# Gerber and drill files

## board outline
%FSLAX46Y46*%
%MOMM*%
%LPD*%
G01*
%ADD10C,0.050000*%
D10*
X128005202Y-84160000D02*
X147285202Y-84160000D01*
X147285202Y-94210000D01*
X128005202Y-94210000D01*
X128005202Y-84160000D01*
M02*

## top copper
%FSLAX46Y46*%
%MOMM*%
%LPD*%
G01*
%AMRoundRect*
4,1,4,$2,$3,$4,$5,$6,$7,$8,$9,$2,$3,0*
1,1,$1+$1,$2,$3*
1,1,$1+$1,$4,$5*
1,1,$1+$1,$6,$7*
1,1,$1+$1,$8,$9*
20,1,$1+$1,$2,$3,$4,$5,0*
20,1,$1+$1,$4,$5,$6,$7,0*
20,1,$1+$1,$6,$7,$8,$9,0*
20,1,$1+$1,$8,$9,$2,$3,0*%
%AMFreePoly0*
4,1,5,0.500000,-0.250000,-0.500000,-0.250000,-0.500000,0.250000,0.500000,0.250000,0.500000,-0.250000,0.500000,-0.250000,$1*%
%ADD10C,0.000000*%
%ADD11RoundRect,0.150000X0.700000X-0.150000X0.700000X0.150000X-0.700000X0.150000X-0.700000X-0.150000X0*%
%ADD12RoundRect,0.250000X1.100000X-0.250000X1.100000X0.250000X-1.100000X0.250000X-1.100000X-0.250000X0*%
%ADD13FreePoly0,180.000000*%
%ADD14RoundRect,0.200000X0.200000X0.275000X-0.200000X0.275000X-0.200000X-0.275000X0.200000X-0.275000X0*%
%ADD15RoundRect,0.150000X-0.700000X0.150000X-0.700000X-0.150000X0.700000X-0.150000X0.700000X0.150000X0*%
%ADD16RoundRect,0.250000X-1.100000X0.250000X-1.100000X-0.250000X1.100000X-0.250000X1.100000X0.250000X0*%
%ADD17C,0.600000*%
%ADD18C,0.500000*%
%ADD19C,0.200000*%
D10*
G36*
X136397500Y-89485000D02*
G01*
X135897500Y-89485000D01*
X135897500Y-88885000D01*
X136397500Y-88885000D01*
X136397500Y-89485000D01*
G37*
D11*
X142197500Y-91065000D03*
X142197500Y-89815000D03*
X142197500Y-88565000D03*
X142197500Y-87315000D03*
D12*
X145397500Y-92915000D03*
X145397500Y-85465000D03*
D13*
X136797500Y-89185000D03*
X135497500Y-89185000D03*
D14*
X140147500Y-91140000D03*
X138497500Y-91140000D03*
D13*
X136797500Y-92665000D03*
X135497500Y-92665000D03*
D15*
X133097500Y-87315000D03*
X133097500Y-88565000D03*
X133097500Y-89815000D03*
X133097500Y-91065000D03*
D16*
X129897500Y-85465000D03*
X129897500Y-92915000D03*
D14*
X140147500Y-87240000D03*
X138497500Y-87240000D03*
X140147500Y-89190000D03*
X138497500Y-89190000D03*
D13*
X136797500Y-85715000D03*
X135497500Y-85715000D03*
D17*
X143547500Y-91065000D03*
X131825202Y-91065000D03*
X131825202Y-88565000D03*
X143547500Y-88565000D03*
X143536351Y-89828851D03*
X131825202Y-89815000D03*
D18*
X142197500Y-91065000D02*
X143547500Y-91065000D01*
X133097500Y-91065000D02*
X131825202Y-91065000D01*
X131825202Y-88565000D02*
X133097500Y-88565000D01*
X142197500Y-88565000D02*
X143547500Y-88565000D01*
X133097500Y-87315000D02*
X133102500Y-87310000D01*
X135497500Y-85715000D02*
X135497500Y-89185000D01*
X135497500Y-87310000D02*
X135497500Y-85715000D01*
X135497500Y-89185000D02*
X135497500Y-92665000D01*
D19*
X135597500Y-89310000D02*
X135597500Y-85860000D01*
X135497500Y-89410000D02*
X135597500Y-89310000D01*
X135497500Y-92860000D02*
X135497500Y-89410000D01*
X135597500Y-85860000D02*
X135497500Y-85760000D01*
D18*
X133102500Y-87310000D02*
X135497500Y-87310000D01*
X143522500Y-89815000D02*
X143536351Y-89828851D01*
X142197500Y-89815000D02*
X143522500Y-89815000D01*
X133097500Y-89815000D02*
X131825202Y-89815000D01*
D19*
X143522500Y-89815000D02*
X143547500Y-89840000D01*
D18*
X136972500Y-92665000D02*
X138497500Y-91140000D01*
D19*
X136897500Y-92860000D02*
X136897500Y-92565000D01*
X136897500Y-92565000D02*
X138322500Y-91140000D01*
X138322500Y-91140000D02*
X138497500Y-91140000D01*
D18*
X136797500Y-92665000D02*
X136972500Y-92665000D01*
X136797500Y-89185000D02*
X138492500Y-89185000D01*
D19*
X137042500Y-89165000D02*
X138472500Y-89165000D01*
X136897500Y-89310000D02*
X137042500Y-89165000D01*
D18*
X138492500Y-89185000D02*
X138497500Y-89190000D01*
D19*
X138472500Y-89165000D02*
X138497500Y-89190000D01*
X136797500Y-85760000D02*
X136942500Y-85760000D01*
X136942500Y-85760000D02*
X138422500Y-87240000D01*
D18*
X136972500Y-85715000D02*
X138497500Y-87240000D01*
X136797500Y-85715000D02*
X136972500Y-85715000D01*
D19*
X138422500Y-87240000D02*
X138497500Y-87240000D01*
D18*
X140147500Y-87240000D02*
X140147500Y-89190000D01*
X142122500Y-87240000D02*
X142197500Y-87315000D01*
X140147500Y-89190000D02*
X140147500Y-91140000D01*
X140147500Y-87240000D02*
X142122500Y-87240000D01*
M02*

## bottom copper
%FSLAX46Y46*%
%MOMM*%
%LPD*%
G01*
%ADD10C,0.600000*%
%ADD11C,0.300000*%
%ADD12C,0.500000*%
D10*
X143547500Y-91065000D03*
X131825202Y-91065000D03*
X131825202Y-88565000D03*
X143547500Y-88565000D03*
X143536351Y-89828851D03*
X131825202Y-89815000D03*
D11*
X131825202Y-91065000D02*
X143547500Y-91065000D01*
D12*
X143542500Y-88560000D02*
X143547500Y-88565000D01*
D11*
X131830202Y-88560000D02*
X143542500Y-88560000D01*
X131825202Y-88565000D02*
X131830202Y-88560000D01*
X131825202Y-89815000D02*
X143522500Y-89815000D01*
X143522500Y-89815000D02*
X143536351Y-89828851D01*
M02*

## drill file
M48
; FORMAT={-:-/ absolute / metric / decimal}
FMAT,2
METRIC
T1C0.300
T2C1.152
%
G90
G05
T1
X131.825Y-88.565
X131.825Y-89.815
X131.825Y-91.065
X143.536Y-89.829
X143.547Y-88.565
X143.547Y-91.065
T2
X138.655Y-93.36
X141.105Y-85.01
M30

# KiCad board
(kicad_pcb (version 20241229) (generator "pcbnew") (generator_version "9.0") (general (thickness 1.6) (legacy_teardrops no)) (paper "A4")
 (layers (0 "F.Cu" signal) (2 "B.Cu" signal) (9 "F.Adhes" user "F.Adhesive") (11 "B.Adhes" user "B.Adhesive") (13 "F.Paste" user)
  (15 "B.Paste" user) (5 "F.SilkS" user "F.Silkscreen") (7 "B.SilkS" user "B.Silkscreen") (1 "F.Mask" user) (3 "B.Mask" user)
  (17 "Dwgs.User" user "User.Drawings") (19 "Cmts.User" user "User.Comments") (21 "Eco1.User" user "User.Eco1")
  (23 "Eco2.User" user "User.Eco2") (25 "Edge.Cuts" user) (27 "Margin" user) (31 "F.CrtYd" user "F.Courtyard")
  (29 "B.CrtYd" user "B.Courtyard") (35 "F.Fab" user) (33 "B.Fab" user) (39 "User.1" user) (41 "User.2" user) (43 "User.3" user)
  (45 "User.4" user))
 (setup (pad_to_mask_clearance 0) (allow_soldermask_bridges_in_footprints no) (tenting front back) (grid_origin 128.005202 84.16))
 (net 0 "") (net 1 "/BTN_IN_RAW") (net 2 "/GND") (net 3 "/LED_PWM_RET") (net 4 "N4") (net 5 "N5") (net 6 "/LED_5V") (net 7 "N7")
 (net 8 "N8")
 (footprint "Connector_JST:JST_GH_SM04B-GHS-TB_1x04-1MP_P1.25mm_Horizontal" (layer "F.Cu") (at 144.0475 89.19 90)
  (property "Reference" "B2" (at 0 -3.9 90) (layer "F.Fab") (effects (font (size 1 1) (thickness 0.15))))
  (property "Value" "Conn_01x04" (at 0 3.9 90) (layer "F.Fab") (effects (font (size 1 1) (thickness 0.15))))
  (pad "1" smd roundrect (at -1.875 -1.85 90) (size 0.6 1.7) (layers "F.Cu" "F.Mask" "F.Paste") (roundrect_rratio 0.25)
   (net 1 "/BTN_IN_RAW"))
  (pad "2" smd roundrect (at -0.625 -1.85 90) (size 0.6 1.7) (layers "F.Cu" "F.Mask" "F.Paste") (roundrect_rratio 0.25) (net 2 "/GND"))
  (pad "3" smd roundrect (at 0.625 -1.85 90) (size 0.6 1.7) (layers "F.Cu" "F.Mask" "F.Paste") (roundrect_rratio 0.25)
   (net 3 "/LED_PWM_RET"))
  (pad "4" smd roundrect (at 1.875 -1.85 90) (size 0.6 1.7) (layers "F.Cu" "F.Mask" "F.Paste") (roundrect_rratio 0.25) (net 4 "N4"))
  (pad "MP" smd roundrect (at -3.725 1.35 90) (size 1 2.7) (layers "F.Cu" "F.Mask" "F.Paste") (roundrect_rratio 0.25))
  (pad "MP" smd roundrect (at 3.725 1.35 90) (size 1 2.7) (layers "F.Cu" "F.Mask" "F.Paste") (roundrect_rratio 0.25)))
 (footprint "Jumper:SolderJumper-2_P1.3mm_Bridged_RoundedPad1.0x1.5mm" (layer "F.Cu") (at 136.1475 89.185 180)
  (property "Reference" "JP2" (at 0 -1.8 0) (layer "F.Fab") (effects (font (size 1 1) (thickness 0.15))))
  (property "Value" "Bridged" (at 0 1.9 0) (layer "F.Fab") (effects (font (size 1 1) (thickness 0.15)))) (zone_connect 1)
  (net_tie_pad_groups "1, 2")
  (fp_poly (pts (xy 0.25 -0.3) (xy -0.25 -0.3) (xy -0.25 0.3) (xy 0.25 0.3)) (stroke (width 0) (type solid)) (fill yes) (layer "F.Cu"))
  (pad "1" smd custom (at -0.65 0 180) (size 1 0.5) (layers "F.Cu" "F.Mask") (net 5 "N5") (zone_connect 2) (thermal_bridge_angle 45)
   (options (clearance outline) (anchor rect)) (primitives))
  (pad "2" smd custom (at 0.65 0 180) (size 1 0.5) (layers "F.Cu" "F.Mask") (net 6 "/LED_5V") (zone_connect 2) (thermal_bridge_angle 45)
   (options (clearance outline) (anchor rect)) (primitives)))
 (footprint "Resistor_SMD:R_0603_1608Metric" (layer "F.Cu") (at 139.3225 91.14 180)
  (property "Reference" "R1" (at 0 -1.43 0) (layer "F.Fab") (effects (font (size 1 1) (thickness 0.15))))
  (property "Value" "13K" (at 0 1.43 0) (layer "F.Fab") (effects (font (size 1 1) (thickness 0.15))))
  (pad "1" smd roundrect (at -0.825 0 180) (size 0.8 0.95) (layers "F.Cu" "F.Mask" "F.Paste") (roundrect_rratio 0.25) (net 4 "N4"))
  (pad "2" smd roundrect (at 0.825 0 180) (size 0.8 0.95) (layers "F.Cu" "F.Mask" "F.Paste") (roundrect_rratio 0.25) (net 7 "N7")))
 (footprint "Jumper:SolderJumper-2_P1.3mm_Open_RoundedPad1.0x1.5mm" (layer "F.Cu") (at 136.1475 92.665 180)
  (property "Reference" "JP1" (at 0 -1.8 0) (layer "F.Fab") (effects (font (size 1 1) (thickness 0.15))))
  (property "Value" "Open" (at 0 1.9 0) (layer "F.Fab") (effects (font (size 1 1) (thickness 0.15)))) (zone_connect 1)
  (pad "1" smd custom (at -0.65 0 180) (size 1 0.5) (layers "F.Cu" "F.Mask") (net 7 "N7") (zone_connect 2) (thermal_bridge_angle 45)
   (options (clearance outline) (anchor rect)) (primitives))
  (pad "2" smd custom (at 0.65 0 180) (size 1 0.5) (layers "F.Cu" "F.Mask") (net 6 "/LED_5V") (zone_connect 2) (thermal_bridge_angle 45)
   (options (clearance outline) (anchor rect)) (primitives)))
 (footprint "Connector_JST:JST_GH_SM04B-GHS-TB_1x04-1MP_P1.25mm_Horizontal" (layer "F.Cu") (at 131.2475 89.19 -90)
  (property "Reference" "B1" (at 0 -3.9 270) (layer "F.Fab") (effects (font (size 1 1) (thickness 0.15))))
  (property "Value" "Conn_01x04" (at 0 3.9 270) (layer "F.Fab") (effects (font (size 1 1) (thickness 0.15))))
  (pad "1" smd roundrect (at -1.875 -1.85 270) (size 0.6 1.7) (layers "F.Cu" "F.Mask" "F.Paste") (roundrect_rratio 0.25) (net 6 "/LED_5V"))
  (pad "2" smd roundrect (at -0.625 -1.85 270) (size 0.6 1.7) (layers "F.Cu" "F.Mask" "F.Paste") (roundrect_rratio 0.25)
   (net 3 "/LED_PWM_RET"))
  (pad "3" smd roundrect (at 0.625 -1.85 270) (size 0.6 1.7) (layers "F.Cu" "F.Mask" "F.Paste") (roundrect_rratio 0.25) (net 2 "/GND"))
  (pad "4" smd roundrect (at 1.875 -1.85 270) (size 0.6 1.7) (layers "F.Cu" "F.Mask" "F.Paste") (roundrect_rratio 0.25)
   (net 1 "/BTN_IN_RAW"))
  (pad "MP" smd roundrect (at -3.725 1.35 270) (size 1 2.7) (layers "F.Cu" "F.Mask" "F.Paste") (roundrect_rratio 0.25))
  (pad "MP" smd roundrect (at 3.725 1.35 270) (size 1 2.7) (layers "F.Cu" "F.Mask" "F.Paste") (roundrect_rratio 0.25)))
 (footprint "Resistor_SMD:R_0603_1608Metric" (layer "F.Cu") (at 139.3225 87.24 180)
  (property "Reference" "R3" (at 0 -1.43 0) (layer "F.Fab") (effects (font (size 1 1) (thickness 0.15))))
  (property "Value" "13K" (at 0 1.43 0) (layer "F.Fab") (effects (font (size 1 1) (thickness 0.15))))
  (pad "1" smd roundrect (at -0.825 0 180) (size 0.8 0.95) (layers "F.Cu" "F.Mask" "F.Paste") (roundrect_rratio 0.25) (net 4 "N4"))
  (pad "2" smd roundrect (at 0.825 0 180) (size 0.8 0.95) (layers "F.Cu" "F.Mask" "F.Paste") (roundrect_rratio 0.25) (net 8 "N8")))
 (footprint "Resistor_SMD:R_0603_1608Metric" (layer "F.Cu") (at 139.3225 89.19 180)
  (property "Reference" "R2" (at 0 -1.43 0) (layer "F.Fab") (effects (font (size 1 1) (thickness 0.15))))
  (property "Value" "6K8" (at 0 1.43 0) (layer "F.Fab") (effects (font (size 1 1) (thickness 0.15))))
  (pad "1" smd roundrect (at -0.825 0 180) (size 0.8 0.95) (layers "F.Cu" "F.Mask" "F.Paste") (roundrect_rratio 0.25) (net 4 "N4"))
  (pad "2" smd roundrect (at 0.825 0 180) (size 0.8 0.95) (layers "F.Cu" "F.Mask" "F.Paste") (roundrect_rratio 0.25) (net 5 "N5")))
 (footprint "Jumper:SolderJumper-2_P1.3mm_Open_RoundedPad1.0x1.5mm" (layer "F.Cu") (at 136.1475 85.715 180)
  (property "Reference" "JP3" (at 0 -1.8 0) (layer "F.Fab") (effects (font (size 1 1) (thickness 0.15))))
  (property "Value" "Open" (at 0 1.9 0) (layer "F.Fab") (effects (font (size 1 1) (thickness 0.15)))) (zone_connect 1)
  (pad "1" smd custom (at -0.65 0 180) (size 1 0.5) (layers "F.Cu" "F.Mask") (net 8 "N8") (zone_connect 2) (thermal_bridge_angle 45)
   (options (clearance outline) (anchor rect)) (primitives))
  (pad "2" smd custom (at 0.65 0 180) (size 1 0.5) (layers "F.Cu" "F.Mask") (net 6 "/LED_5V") (zone_connect 2) (thermal_bridge_angle 45)
   (options (clearance outline) (anchor rect)) (primitives)))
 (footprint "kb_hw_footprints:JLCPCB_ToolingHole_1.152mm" (layer "B.Cu") (at 138.655202 93.36 180)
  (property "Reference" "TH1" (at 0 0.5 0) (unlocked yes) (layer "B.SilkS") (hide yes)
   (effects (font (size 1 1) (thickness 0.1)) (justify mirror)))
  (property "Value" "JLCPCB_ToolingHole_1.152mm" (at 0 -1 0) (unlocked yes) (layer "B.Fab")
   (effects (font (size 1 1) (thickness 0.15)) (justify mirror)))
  (pad "" np_thru_hole circle (at 0 0 180) (size 1.152 1.152) (drill 1.152) (layers "*.Cu" "*.Mask") (solder_mask_margin 0.148)
   (clearance 0.25) (thermal_bridge_angle 90)))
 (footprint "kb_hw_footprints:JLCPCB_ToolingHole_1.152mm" (layer "B.Cu") (at 141.105202 85.01 180)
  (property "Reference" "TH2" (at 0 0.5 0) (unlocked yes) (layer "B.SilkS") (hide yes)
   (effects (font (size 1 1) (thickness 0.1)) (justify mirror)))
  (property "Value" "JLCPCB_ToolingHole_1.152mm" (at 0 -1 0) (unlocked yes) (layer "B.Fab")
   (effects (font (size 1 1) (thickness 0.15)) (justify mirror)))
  (pad "" np_thru_hole circle (at 0 0 180) (size 1.152 1.152) (drill 1.152) (layers "*.Cu" "*.Mask") (solder_mask_margin 0.148)
   (clearance 0.25) (thermal_bridge_angle 90)))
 (gr_rect (start 128.005202 84.16) (end 147.285202 94.21) (stroke (width 0.05) (type solid)) (fill no) (layer "Edge.Cuts"))
 (segment (start 142.1975 91.065) (end 143.5475 91.065) (width 0.5) (layer "F.Cu") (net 1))
 (segment (start 133.0975 91.065) (end 131.825202 91.065) (width 0.5) (layer "F.Cu") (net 1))
 (via (at 143.5475 91.065) (size 0.6) (drill 0.3) (layers "F.Cu" "B.Cu") (free yes) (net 1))
 (via (at 131.825202 91.065) (size 0.6) (drill 0.3) (layers "F.Cu" "B.Cu") (free yes) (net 1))
 (segment (start 131.825202 91.065) (end 143.5475 91.065) (width 0.3) (layer "B.Cu") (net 1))
 (segment (start 131.825202 88.565) (end 133.0975 88.565) (width 0.5) (layer "F.Cu") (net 3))
 (segment (start 142.1975 88.565) (end 143.5475 88.565) (width 0.5) (layer "F.Cu") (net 3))
 (via (at 131.825202 88.565) (size 0.6) (drill 0.3) (layers "F.Cu" "B.Cu") (free yes) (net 3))
 (via (at 143.5475 88.565) (size 0.6) (drill 0.3) (layers "F.Cu" "B.Cu") (free yes) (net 3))
 (segment (start 143.5425 88.56) (end 143.5475 88.565) (width 0.5) (layer "B.Cu") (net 3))
 (segment (start 131.830202 88.56) (end 143.5425 88.56) (width 0.3) (layer "B.Cu") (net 3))
 (segment (start 131.825202 88.565) (end 131.830202 88.56) (width 0.3) (layer "B.Cu") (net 3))
 (segment (start 133.0975 87.315) (end 133.1025 87.31) (width 0.5) (layer "F.Cu") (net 6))
 (segment (start 135.4975 85.715) (end 135.4975 89.185) (width 0.5) (layer "F.Cu") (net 6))
 (segment (start 135.4975 87.31) (end 135.4975 85.715) (width 0.5) (layer "F.Cu") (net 6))
 (segment (start 135.4975 89.185) (end 135.4975 92.665) (width 0.5) (layer "F.Cu") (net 6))
 (segment (start 135.5975 89.31) (end 135.5975 85.86) (width 0.2) (layer "F.Cu") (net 6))
 (segment (start 135.4975 89.41) (end 135.5975 89.31) (width 0.2) (layer "F.Cu") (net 6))
 (segment (start 135.4975 92.86) (end 135.4975 89.41) (width 0.2) (layer "F.Cu") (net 6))
 (segment (start 135.5975 85.86) (end 135.4975 85.76) (width 0.2) (layer "F.Cu") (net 6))
 (segment (start 133.1025 87.31) (end 135.4975 87.31) (width 0.5) (layer "F.Cu") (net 6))
 (segment (start 143.5225 89.815) (end 143.536351 89.828851) (width 0.5) (layer "F.Cu") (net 2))
 (segment (start 142.1975 89.815) (end 143.5225 89.815) (width 0.5) (layer "F.Cu") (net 2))
 (segment (start 133.0975 89.815) (end 131.825202 89.815) (width 0.5) (layer "F.Cu") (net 2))
 (segment (start 143.5225 89.815) (end 143.5475 89.84) (width 0.2) (layer "F.Cu") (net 2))
 (via (at 143.536351 89.828851) (size 0.6) (drill 0.3) (layers "F.Cu" "B.Cu") (free yes) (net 2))
 (via (at 131.825202 89.815) (size 0.6) (drill 0.3) (layers "F.Cu" "B.Cu") (free yes) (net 2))
 (segment (start 131.825202 89.815) (end 143.5225 89.815) (width 0.3) (layer "B.Cu") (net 2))
 (segment (start 143.5225 89.815) (end 143.536351 89.828851) (width 0.3) (layer "B.Cu") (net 2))
 (segment (start 136.9725 92.665) (end 138.4975 91.14) (width 0.5) (layer "F.Cu") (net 7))
 (segment (start 136.8975 92.86) (end 136.8975 92.565) (width 0.2) (layer "F.Cu") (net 7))
 (segment (start 136.8975 92.565) (end 138.3225 91.14) (width 0.2) (layer "F.Cu") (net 7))
 (segment (start 138.3225 91.14) (end 138.4975 91.14) (width 0.2) (layer "F.Cu") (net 7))
 (segment (start 136.7975 92.665) (end 136.9725 92.665) (width 0.5) (layer "F.Cu") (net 7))
 (segment (start 136.7975 89.185) (end 138.4925 89.185) (width 0.5) (layer "F.Cu") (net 5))
 (segment (start 137.0425 89.165) (end 138.4725 89.165) (width 0.2) (layer "F.Cu") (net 5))
 (segment (start 136.8975 89.31) (end 137.0425 89.165) (width 0.2) (layer "F.Cu") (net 5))
 (segment (start 138.4925 89.185) (end 138.4975 89.19) (width 0.5) (layer "F.Cu") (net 5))
 (segment (start 138.4725 89.165) (end 138.4975 89.19) (width 0.2) (layer "F.Cu") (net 5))
 (segment (start 136.7975 85.76) (end 136.9425 85.76) (width 0.2) (layer "F.Cu") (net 8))
 (segment (start 136.9425 85.76) (end 138.4225 87.24) (width 0.2) (layer "F.Cu") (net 8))
 (segment (start 136.9725 85.715) (end 138.4975 87.24) (width 0.5) (layer "F.Cu") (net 8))
 (segment (start 136.7975 85.715) (end 136.9725 85.715) (width 0.5) (layer "F.Cu") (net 8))
 (segment (start 138.4225 87.24) (end 138.4975 87.24) (width 0.2) (layer "F.Cu") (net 8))
 (segment (start 140.1475 87.24) (end 140.1475 89.19) (width 0.5) (layer "F.Cu") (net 4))
 (segment (start 142.1225 87.24) (end 142.1975 87.315) (width 0.5) (layer "F.Cu") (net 4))
 (segment (start 140.1475 89.19) (end 140.1475 91.14) (width 0.5) (layer "F.Cu") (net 4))
 (segment (start 140.1475 87.24) (end 142.1225 87.24) (width 0.5) (layer "F.Cu") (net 4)))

